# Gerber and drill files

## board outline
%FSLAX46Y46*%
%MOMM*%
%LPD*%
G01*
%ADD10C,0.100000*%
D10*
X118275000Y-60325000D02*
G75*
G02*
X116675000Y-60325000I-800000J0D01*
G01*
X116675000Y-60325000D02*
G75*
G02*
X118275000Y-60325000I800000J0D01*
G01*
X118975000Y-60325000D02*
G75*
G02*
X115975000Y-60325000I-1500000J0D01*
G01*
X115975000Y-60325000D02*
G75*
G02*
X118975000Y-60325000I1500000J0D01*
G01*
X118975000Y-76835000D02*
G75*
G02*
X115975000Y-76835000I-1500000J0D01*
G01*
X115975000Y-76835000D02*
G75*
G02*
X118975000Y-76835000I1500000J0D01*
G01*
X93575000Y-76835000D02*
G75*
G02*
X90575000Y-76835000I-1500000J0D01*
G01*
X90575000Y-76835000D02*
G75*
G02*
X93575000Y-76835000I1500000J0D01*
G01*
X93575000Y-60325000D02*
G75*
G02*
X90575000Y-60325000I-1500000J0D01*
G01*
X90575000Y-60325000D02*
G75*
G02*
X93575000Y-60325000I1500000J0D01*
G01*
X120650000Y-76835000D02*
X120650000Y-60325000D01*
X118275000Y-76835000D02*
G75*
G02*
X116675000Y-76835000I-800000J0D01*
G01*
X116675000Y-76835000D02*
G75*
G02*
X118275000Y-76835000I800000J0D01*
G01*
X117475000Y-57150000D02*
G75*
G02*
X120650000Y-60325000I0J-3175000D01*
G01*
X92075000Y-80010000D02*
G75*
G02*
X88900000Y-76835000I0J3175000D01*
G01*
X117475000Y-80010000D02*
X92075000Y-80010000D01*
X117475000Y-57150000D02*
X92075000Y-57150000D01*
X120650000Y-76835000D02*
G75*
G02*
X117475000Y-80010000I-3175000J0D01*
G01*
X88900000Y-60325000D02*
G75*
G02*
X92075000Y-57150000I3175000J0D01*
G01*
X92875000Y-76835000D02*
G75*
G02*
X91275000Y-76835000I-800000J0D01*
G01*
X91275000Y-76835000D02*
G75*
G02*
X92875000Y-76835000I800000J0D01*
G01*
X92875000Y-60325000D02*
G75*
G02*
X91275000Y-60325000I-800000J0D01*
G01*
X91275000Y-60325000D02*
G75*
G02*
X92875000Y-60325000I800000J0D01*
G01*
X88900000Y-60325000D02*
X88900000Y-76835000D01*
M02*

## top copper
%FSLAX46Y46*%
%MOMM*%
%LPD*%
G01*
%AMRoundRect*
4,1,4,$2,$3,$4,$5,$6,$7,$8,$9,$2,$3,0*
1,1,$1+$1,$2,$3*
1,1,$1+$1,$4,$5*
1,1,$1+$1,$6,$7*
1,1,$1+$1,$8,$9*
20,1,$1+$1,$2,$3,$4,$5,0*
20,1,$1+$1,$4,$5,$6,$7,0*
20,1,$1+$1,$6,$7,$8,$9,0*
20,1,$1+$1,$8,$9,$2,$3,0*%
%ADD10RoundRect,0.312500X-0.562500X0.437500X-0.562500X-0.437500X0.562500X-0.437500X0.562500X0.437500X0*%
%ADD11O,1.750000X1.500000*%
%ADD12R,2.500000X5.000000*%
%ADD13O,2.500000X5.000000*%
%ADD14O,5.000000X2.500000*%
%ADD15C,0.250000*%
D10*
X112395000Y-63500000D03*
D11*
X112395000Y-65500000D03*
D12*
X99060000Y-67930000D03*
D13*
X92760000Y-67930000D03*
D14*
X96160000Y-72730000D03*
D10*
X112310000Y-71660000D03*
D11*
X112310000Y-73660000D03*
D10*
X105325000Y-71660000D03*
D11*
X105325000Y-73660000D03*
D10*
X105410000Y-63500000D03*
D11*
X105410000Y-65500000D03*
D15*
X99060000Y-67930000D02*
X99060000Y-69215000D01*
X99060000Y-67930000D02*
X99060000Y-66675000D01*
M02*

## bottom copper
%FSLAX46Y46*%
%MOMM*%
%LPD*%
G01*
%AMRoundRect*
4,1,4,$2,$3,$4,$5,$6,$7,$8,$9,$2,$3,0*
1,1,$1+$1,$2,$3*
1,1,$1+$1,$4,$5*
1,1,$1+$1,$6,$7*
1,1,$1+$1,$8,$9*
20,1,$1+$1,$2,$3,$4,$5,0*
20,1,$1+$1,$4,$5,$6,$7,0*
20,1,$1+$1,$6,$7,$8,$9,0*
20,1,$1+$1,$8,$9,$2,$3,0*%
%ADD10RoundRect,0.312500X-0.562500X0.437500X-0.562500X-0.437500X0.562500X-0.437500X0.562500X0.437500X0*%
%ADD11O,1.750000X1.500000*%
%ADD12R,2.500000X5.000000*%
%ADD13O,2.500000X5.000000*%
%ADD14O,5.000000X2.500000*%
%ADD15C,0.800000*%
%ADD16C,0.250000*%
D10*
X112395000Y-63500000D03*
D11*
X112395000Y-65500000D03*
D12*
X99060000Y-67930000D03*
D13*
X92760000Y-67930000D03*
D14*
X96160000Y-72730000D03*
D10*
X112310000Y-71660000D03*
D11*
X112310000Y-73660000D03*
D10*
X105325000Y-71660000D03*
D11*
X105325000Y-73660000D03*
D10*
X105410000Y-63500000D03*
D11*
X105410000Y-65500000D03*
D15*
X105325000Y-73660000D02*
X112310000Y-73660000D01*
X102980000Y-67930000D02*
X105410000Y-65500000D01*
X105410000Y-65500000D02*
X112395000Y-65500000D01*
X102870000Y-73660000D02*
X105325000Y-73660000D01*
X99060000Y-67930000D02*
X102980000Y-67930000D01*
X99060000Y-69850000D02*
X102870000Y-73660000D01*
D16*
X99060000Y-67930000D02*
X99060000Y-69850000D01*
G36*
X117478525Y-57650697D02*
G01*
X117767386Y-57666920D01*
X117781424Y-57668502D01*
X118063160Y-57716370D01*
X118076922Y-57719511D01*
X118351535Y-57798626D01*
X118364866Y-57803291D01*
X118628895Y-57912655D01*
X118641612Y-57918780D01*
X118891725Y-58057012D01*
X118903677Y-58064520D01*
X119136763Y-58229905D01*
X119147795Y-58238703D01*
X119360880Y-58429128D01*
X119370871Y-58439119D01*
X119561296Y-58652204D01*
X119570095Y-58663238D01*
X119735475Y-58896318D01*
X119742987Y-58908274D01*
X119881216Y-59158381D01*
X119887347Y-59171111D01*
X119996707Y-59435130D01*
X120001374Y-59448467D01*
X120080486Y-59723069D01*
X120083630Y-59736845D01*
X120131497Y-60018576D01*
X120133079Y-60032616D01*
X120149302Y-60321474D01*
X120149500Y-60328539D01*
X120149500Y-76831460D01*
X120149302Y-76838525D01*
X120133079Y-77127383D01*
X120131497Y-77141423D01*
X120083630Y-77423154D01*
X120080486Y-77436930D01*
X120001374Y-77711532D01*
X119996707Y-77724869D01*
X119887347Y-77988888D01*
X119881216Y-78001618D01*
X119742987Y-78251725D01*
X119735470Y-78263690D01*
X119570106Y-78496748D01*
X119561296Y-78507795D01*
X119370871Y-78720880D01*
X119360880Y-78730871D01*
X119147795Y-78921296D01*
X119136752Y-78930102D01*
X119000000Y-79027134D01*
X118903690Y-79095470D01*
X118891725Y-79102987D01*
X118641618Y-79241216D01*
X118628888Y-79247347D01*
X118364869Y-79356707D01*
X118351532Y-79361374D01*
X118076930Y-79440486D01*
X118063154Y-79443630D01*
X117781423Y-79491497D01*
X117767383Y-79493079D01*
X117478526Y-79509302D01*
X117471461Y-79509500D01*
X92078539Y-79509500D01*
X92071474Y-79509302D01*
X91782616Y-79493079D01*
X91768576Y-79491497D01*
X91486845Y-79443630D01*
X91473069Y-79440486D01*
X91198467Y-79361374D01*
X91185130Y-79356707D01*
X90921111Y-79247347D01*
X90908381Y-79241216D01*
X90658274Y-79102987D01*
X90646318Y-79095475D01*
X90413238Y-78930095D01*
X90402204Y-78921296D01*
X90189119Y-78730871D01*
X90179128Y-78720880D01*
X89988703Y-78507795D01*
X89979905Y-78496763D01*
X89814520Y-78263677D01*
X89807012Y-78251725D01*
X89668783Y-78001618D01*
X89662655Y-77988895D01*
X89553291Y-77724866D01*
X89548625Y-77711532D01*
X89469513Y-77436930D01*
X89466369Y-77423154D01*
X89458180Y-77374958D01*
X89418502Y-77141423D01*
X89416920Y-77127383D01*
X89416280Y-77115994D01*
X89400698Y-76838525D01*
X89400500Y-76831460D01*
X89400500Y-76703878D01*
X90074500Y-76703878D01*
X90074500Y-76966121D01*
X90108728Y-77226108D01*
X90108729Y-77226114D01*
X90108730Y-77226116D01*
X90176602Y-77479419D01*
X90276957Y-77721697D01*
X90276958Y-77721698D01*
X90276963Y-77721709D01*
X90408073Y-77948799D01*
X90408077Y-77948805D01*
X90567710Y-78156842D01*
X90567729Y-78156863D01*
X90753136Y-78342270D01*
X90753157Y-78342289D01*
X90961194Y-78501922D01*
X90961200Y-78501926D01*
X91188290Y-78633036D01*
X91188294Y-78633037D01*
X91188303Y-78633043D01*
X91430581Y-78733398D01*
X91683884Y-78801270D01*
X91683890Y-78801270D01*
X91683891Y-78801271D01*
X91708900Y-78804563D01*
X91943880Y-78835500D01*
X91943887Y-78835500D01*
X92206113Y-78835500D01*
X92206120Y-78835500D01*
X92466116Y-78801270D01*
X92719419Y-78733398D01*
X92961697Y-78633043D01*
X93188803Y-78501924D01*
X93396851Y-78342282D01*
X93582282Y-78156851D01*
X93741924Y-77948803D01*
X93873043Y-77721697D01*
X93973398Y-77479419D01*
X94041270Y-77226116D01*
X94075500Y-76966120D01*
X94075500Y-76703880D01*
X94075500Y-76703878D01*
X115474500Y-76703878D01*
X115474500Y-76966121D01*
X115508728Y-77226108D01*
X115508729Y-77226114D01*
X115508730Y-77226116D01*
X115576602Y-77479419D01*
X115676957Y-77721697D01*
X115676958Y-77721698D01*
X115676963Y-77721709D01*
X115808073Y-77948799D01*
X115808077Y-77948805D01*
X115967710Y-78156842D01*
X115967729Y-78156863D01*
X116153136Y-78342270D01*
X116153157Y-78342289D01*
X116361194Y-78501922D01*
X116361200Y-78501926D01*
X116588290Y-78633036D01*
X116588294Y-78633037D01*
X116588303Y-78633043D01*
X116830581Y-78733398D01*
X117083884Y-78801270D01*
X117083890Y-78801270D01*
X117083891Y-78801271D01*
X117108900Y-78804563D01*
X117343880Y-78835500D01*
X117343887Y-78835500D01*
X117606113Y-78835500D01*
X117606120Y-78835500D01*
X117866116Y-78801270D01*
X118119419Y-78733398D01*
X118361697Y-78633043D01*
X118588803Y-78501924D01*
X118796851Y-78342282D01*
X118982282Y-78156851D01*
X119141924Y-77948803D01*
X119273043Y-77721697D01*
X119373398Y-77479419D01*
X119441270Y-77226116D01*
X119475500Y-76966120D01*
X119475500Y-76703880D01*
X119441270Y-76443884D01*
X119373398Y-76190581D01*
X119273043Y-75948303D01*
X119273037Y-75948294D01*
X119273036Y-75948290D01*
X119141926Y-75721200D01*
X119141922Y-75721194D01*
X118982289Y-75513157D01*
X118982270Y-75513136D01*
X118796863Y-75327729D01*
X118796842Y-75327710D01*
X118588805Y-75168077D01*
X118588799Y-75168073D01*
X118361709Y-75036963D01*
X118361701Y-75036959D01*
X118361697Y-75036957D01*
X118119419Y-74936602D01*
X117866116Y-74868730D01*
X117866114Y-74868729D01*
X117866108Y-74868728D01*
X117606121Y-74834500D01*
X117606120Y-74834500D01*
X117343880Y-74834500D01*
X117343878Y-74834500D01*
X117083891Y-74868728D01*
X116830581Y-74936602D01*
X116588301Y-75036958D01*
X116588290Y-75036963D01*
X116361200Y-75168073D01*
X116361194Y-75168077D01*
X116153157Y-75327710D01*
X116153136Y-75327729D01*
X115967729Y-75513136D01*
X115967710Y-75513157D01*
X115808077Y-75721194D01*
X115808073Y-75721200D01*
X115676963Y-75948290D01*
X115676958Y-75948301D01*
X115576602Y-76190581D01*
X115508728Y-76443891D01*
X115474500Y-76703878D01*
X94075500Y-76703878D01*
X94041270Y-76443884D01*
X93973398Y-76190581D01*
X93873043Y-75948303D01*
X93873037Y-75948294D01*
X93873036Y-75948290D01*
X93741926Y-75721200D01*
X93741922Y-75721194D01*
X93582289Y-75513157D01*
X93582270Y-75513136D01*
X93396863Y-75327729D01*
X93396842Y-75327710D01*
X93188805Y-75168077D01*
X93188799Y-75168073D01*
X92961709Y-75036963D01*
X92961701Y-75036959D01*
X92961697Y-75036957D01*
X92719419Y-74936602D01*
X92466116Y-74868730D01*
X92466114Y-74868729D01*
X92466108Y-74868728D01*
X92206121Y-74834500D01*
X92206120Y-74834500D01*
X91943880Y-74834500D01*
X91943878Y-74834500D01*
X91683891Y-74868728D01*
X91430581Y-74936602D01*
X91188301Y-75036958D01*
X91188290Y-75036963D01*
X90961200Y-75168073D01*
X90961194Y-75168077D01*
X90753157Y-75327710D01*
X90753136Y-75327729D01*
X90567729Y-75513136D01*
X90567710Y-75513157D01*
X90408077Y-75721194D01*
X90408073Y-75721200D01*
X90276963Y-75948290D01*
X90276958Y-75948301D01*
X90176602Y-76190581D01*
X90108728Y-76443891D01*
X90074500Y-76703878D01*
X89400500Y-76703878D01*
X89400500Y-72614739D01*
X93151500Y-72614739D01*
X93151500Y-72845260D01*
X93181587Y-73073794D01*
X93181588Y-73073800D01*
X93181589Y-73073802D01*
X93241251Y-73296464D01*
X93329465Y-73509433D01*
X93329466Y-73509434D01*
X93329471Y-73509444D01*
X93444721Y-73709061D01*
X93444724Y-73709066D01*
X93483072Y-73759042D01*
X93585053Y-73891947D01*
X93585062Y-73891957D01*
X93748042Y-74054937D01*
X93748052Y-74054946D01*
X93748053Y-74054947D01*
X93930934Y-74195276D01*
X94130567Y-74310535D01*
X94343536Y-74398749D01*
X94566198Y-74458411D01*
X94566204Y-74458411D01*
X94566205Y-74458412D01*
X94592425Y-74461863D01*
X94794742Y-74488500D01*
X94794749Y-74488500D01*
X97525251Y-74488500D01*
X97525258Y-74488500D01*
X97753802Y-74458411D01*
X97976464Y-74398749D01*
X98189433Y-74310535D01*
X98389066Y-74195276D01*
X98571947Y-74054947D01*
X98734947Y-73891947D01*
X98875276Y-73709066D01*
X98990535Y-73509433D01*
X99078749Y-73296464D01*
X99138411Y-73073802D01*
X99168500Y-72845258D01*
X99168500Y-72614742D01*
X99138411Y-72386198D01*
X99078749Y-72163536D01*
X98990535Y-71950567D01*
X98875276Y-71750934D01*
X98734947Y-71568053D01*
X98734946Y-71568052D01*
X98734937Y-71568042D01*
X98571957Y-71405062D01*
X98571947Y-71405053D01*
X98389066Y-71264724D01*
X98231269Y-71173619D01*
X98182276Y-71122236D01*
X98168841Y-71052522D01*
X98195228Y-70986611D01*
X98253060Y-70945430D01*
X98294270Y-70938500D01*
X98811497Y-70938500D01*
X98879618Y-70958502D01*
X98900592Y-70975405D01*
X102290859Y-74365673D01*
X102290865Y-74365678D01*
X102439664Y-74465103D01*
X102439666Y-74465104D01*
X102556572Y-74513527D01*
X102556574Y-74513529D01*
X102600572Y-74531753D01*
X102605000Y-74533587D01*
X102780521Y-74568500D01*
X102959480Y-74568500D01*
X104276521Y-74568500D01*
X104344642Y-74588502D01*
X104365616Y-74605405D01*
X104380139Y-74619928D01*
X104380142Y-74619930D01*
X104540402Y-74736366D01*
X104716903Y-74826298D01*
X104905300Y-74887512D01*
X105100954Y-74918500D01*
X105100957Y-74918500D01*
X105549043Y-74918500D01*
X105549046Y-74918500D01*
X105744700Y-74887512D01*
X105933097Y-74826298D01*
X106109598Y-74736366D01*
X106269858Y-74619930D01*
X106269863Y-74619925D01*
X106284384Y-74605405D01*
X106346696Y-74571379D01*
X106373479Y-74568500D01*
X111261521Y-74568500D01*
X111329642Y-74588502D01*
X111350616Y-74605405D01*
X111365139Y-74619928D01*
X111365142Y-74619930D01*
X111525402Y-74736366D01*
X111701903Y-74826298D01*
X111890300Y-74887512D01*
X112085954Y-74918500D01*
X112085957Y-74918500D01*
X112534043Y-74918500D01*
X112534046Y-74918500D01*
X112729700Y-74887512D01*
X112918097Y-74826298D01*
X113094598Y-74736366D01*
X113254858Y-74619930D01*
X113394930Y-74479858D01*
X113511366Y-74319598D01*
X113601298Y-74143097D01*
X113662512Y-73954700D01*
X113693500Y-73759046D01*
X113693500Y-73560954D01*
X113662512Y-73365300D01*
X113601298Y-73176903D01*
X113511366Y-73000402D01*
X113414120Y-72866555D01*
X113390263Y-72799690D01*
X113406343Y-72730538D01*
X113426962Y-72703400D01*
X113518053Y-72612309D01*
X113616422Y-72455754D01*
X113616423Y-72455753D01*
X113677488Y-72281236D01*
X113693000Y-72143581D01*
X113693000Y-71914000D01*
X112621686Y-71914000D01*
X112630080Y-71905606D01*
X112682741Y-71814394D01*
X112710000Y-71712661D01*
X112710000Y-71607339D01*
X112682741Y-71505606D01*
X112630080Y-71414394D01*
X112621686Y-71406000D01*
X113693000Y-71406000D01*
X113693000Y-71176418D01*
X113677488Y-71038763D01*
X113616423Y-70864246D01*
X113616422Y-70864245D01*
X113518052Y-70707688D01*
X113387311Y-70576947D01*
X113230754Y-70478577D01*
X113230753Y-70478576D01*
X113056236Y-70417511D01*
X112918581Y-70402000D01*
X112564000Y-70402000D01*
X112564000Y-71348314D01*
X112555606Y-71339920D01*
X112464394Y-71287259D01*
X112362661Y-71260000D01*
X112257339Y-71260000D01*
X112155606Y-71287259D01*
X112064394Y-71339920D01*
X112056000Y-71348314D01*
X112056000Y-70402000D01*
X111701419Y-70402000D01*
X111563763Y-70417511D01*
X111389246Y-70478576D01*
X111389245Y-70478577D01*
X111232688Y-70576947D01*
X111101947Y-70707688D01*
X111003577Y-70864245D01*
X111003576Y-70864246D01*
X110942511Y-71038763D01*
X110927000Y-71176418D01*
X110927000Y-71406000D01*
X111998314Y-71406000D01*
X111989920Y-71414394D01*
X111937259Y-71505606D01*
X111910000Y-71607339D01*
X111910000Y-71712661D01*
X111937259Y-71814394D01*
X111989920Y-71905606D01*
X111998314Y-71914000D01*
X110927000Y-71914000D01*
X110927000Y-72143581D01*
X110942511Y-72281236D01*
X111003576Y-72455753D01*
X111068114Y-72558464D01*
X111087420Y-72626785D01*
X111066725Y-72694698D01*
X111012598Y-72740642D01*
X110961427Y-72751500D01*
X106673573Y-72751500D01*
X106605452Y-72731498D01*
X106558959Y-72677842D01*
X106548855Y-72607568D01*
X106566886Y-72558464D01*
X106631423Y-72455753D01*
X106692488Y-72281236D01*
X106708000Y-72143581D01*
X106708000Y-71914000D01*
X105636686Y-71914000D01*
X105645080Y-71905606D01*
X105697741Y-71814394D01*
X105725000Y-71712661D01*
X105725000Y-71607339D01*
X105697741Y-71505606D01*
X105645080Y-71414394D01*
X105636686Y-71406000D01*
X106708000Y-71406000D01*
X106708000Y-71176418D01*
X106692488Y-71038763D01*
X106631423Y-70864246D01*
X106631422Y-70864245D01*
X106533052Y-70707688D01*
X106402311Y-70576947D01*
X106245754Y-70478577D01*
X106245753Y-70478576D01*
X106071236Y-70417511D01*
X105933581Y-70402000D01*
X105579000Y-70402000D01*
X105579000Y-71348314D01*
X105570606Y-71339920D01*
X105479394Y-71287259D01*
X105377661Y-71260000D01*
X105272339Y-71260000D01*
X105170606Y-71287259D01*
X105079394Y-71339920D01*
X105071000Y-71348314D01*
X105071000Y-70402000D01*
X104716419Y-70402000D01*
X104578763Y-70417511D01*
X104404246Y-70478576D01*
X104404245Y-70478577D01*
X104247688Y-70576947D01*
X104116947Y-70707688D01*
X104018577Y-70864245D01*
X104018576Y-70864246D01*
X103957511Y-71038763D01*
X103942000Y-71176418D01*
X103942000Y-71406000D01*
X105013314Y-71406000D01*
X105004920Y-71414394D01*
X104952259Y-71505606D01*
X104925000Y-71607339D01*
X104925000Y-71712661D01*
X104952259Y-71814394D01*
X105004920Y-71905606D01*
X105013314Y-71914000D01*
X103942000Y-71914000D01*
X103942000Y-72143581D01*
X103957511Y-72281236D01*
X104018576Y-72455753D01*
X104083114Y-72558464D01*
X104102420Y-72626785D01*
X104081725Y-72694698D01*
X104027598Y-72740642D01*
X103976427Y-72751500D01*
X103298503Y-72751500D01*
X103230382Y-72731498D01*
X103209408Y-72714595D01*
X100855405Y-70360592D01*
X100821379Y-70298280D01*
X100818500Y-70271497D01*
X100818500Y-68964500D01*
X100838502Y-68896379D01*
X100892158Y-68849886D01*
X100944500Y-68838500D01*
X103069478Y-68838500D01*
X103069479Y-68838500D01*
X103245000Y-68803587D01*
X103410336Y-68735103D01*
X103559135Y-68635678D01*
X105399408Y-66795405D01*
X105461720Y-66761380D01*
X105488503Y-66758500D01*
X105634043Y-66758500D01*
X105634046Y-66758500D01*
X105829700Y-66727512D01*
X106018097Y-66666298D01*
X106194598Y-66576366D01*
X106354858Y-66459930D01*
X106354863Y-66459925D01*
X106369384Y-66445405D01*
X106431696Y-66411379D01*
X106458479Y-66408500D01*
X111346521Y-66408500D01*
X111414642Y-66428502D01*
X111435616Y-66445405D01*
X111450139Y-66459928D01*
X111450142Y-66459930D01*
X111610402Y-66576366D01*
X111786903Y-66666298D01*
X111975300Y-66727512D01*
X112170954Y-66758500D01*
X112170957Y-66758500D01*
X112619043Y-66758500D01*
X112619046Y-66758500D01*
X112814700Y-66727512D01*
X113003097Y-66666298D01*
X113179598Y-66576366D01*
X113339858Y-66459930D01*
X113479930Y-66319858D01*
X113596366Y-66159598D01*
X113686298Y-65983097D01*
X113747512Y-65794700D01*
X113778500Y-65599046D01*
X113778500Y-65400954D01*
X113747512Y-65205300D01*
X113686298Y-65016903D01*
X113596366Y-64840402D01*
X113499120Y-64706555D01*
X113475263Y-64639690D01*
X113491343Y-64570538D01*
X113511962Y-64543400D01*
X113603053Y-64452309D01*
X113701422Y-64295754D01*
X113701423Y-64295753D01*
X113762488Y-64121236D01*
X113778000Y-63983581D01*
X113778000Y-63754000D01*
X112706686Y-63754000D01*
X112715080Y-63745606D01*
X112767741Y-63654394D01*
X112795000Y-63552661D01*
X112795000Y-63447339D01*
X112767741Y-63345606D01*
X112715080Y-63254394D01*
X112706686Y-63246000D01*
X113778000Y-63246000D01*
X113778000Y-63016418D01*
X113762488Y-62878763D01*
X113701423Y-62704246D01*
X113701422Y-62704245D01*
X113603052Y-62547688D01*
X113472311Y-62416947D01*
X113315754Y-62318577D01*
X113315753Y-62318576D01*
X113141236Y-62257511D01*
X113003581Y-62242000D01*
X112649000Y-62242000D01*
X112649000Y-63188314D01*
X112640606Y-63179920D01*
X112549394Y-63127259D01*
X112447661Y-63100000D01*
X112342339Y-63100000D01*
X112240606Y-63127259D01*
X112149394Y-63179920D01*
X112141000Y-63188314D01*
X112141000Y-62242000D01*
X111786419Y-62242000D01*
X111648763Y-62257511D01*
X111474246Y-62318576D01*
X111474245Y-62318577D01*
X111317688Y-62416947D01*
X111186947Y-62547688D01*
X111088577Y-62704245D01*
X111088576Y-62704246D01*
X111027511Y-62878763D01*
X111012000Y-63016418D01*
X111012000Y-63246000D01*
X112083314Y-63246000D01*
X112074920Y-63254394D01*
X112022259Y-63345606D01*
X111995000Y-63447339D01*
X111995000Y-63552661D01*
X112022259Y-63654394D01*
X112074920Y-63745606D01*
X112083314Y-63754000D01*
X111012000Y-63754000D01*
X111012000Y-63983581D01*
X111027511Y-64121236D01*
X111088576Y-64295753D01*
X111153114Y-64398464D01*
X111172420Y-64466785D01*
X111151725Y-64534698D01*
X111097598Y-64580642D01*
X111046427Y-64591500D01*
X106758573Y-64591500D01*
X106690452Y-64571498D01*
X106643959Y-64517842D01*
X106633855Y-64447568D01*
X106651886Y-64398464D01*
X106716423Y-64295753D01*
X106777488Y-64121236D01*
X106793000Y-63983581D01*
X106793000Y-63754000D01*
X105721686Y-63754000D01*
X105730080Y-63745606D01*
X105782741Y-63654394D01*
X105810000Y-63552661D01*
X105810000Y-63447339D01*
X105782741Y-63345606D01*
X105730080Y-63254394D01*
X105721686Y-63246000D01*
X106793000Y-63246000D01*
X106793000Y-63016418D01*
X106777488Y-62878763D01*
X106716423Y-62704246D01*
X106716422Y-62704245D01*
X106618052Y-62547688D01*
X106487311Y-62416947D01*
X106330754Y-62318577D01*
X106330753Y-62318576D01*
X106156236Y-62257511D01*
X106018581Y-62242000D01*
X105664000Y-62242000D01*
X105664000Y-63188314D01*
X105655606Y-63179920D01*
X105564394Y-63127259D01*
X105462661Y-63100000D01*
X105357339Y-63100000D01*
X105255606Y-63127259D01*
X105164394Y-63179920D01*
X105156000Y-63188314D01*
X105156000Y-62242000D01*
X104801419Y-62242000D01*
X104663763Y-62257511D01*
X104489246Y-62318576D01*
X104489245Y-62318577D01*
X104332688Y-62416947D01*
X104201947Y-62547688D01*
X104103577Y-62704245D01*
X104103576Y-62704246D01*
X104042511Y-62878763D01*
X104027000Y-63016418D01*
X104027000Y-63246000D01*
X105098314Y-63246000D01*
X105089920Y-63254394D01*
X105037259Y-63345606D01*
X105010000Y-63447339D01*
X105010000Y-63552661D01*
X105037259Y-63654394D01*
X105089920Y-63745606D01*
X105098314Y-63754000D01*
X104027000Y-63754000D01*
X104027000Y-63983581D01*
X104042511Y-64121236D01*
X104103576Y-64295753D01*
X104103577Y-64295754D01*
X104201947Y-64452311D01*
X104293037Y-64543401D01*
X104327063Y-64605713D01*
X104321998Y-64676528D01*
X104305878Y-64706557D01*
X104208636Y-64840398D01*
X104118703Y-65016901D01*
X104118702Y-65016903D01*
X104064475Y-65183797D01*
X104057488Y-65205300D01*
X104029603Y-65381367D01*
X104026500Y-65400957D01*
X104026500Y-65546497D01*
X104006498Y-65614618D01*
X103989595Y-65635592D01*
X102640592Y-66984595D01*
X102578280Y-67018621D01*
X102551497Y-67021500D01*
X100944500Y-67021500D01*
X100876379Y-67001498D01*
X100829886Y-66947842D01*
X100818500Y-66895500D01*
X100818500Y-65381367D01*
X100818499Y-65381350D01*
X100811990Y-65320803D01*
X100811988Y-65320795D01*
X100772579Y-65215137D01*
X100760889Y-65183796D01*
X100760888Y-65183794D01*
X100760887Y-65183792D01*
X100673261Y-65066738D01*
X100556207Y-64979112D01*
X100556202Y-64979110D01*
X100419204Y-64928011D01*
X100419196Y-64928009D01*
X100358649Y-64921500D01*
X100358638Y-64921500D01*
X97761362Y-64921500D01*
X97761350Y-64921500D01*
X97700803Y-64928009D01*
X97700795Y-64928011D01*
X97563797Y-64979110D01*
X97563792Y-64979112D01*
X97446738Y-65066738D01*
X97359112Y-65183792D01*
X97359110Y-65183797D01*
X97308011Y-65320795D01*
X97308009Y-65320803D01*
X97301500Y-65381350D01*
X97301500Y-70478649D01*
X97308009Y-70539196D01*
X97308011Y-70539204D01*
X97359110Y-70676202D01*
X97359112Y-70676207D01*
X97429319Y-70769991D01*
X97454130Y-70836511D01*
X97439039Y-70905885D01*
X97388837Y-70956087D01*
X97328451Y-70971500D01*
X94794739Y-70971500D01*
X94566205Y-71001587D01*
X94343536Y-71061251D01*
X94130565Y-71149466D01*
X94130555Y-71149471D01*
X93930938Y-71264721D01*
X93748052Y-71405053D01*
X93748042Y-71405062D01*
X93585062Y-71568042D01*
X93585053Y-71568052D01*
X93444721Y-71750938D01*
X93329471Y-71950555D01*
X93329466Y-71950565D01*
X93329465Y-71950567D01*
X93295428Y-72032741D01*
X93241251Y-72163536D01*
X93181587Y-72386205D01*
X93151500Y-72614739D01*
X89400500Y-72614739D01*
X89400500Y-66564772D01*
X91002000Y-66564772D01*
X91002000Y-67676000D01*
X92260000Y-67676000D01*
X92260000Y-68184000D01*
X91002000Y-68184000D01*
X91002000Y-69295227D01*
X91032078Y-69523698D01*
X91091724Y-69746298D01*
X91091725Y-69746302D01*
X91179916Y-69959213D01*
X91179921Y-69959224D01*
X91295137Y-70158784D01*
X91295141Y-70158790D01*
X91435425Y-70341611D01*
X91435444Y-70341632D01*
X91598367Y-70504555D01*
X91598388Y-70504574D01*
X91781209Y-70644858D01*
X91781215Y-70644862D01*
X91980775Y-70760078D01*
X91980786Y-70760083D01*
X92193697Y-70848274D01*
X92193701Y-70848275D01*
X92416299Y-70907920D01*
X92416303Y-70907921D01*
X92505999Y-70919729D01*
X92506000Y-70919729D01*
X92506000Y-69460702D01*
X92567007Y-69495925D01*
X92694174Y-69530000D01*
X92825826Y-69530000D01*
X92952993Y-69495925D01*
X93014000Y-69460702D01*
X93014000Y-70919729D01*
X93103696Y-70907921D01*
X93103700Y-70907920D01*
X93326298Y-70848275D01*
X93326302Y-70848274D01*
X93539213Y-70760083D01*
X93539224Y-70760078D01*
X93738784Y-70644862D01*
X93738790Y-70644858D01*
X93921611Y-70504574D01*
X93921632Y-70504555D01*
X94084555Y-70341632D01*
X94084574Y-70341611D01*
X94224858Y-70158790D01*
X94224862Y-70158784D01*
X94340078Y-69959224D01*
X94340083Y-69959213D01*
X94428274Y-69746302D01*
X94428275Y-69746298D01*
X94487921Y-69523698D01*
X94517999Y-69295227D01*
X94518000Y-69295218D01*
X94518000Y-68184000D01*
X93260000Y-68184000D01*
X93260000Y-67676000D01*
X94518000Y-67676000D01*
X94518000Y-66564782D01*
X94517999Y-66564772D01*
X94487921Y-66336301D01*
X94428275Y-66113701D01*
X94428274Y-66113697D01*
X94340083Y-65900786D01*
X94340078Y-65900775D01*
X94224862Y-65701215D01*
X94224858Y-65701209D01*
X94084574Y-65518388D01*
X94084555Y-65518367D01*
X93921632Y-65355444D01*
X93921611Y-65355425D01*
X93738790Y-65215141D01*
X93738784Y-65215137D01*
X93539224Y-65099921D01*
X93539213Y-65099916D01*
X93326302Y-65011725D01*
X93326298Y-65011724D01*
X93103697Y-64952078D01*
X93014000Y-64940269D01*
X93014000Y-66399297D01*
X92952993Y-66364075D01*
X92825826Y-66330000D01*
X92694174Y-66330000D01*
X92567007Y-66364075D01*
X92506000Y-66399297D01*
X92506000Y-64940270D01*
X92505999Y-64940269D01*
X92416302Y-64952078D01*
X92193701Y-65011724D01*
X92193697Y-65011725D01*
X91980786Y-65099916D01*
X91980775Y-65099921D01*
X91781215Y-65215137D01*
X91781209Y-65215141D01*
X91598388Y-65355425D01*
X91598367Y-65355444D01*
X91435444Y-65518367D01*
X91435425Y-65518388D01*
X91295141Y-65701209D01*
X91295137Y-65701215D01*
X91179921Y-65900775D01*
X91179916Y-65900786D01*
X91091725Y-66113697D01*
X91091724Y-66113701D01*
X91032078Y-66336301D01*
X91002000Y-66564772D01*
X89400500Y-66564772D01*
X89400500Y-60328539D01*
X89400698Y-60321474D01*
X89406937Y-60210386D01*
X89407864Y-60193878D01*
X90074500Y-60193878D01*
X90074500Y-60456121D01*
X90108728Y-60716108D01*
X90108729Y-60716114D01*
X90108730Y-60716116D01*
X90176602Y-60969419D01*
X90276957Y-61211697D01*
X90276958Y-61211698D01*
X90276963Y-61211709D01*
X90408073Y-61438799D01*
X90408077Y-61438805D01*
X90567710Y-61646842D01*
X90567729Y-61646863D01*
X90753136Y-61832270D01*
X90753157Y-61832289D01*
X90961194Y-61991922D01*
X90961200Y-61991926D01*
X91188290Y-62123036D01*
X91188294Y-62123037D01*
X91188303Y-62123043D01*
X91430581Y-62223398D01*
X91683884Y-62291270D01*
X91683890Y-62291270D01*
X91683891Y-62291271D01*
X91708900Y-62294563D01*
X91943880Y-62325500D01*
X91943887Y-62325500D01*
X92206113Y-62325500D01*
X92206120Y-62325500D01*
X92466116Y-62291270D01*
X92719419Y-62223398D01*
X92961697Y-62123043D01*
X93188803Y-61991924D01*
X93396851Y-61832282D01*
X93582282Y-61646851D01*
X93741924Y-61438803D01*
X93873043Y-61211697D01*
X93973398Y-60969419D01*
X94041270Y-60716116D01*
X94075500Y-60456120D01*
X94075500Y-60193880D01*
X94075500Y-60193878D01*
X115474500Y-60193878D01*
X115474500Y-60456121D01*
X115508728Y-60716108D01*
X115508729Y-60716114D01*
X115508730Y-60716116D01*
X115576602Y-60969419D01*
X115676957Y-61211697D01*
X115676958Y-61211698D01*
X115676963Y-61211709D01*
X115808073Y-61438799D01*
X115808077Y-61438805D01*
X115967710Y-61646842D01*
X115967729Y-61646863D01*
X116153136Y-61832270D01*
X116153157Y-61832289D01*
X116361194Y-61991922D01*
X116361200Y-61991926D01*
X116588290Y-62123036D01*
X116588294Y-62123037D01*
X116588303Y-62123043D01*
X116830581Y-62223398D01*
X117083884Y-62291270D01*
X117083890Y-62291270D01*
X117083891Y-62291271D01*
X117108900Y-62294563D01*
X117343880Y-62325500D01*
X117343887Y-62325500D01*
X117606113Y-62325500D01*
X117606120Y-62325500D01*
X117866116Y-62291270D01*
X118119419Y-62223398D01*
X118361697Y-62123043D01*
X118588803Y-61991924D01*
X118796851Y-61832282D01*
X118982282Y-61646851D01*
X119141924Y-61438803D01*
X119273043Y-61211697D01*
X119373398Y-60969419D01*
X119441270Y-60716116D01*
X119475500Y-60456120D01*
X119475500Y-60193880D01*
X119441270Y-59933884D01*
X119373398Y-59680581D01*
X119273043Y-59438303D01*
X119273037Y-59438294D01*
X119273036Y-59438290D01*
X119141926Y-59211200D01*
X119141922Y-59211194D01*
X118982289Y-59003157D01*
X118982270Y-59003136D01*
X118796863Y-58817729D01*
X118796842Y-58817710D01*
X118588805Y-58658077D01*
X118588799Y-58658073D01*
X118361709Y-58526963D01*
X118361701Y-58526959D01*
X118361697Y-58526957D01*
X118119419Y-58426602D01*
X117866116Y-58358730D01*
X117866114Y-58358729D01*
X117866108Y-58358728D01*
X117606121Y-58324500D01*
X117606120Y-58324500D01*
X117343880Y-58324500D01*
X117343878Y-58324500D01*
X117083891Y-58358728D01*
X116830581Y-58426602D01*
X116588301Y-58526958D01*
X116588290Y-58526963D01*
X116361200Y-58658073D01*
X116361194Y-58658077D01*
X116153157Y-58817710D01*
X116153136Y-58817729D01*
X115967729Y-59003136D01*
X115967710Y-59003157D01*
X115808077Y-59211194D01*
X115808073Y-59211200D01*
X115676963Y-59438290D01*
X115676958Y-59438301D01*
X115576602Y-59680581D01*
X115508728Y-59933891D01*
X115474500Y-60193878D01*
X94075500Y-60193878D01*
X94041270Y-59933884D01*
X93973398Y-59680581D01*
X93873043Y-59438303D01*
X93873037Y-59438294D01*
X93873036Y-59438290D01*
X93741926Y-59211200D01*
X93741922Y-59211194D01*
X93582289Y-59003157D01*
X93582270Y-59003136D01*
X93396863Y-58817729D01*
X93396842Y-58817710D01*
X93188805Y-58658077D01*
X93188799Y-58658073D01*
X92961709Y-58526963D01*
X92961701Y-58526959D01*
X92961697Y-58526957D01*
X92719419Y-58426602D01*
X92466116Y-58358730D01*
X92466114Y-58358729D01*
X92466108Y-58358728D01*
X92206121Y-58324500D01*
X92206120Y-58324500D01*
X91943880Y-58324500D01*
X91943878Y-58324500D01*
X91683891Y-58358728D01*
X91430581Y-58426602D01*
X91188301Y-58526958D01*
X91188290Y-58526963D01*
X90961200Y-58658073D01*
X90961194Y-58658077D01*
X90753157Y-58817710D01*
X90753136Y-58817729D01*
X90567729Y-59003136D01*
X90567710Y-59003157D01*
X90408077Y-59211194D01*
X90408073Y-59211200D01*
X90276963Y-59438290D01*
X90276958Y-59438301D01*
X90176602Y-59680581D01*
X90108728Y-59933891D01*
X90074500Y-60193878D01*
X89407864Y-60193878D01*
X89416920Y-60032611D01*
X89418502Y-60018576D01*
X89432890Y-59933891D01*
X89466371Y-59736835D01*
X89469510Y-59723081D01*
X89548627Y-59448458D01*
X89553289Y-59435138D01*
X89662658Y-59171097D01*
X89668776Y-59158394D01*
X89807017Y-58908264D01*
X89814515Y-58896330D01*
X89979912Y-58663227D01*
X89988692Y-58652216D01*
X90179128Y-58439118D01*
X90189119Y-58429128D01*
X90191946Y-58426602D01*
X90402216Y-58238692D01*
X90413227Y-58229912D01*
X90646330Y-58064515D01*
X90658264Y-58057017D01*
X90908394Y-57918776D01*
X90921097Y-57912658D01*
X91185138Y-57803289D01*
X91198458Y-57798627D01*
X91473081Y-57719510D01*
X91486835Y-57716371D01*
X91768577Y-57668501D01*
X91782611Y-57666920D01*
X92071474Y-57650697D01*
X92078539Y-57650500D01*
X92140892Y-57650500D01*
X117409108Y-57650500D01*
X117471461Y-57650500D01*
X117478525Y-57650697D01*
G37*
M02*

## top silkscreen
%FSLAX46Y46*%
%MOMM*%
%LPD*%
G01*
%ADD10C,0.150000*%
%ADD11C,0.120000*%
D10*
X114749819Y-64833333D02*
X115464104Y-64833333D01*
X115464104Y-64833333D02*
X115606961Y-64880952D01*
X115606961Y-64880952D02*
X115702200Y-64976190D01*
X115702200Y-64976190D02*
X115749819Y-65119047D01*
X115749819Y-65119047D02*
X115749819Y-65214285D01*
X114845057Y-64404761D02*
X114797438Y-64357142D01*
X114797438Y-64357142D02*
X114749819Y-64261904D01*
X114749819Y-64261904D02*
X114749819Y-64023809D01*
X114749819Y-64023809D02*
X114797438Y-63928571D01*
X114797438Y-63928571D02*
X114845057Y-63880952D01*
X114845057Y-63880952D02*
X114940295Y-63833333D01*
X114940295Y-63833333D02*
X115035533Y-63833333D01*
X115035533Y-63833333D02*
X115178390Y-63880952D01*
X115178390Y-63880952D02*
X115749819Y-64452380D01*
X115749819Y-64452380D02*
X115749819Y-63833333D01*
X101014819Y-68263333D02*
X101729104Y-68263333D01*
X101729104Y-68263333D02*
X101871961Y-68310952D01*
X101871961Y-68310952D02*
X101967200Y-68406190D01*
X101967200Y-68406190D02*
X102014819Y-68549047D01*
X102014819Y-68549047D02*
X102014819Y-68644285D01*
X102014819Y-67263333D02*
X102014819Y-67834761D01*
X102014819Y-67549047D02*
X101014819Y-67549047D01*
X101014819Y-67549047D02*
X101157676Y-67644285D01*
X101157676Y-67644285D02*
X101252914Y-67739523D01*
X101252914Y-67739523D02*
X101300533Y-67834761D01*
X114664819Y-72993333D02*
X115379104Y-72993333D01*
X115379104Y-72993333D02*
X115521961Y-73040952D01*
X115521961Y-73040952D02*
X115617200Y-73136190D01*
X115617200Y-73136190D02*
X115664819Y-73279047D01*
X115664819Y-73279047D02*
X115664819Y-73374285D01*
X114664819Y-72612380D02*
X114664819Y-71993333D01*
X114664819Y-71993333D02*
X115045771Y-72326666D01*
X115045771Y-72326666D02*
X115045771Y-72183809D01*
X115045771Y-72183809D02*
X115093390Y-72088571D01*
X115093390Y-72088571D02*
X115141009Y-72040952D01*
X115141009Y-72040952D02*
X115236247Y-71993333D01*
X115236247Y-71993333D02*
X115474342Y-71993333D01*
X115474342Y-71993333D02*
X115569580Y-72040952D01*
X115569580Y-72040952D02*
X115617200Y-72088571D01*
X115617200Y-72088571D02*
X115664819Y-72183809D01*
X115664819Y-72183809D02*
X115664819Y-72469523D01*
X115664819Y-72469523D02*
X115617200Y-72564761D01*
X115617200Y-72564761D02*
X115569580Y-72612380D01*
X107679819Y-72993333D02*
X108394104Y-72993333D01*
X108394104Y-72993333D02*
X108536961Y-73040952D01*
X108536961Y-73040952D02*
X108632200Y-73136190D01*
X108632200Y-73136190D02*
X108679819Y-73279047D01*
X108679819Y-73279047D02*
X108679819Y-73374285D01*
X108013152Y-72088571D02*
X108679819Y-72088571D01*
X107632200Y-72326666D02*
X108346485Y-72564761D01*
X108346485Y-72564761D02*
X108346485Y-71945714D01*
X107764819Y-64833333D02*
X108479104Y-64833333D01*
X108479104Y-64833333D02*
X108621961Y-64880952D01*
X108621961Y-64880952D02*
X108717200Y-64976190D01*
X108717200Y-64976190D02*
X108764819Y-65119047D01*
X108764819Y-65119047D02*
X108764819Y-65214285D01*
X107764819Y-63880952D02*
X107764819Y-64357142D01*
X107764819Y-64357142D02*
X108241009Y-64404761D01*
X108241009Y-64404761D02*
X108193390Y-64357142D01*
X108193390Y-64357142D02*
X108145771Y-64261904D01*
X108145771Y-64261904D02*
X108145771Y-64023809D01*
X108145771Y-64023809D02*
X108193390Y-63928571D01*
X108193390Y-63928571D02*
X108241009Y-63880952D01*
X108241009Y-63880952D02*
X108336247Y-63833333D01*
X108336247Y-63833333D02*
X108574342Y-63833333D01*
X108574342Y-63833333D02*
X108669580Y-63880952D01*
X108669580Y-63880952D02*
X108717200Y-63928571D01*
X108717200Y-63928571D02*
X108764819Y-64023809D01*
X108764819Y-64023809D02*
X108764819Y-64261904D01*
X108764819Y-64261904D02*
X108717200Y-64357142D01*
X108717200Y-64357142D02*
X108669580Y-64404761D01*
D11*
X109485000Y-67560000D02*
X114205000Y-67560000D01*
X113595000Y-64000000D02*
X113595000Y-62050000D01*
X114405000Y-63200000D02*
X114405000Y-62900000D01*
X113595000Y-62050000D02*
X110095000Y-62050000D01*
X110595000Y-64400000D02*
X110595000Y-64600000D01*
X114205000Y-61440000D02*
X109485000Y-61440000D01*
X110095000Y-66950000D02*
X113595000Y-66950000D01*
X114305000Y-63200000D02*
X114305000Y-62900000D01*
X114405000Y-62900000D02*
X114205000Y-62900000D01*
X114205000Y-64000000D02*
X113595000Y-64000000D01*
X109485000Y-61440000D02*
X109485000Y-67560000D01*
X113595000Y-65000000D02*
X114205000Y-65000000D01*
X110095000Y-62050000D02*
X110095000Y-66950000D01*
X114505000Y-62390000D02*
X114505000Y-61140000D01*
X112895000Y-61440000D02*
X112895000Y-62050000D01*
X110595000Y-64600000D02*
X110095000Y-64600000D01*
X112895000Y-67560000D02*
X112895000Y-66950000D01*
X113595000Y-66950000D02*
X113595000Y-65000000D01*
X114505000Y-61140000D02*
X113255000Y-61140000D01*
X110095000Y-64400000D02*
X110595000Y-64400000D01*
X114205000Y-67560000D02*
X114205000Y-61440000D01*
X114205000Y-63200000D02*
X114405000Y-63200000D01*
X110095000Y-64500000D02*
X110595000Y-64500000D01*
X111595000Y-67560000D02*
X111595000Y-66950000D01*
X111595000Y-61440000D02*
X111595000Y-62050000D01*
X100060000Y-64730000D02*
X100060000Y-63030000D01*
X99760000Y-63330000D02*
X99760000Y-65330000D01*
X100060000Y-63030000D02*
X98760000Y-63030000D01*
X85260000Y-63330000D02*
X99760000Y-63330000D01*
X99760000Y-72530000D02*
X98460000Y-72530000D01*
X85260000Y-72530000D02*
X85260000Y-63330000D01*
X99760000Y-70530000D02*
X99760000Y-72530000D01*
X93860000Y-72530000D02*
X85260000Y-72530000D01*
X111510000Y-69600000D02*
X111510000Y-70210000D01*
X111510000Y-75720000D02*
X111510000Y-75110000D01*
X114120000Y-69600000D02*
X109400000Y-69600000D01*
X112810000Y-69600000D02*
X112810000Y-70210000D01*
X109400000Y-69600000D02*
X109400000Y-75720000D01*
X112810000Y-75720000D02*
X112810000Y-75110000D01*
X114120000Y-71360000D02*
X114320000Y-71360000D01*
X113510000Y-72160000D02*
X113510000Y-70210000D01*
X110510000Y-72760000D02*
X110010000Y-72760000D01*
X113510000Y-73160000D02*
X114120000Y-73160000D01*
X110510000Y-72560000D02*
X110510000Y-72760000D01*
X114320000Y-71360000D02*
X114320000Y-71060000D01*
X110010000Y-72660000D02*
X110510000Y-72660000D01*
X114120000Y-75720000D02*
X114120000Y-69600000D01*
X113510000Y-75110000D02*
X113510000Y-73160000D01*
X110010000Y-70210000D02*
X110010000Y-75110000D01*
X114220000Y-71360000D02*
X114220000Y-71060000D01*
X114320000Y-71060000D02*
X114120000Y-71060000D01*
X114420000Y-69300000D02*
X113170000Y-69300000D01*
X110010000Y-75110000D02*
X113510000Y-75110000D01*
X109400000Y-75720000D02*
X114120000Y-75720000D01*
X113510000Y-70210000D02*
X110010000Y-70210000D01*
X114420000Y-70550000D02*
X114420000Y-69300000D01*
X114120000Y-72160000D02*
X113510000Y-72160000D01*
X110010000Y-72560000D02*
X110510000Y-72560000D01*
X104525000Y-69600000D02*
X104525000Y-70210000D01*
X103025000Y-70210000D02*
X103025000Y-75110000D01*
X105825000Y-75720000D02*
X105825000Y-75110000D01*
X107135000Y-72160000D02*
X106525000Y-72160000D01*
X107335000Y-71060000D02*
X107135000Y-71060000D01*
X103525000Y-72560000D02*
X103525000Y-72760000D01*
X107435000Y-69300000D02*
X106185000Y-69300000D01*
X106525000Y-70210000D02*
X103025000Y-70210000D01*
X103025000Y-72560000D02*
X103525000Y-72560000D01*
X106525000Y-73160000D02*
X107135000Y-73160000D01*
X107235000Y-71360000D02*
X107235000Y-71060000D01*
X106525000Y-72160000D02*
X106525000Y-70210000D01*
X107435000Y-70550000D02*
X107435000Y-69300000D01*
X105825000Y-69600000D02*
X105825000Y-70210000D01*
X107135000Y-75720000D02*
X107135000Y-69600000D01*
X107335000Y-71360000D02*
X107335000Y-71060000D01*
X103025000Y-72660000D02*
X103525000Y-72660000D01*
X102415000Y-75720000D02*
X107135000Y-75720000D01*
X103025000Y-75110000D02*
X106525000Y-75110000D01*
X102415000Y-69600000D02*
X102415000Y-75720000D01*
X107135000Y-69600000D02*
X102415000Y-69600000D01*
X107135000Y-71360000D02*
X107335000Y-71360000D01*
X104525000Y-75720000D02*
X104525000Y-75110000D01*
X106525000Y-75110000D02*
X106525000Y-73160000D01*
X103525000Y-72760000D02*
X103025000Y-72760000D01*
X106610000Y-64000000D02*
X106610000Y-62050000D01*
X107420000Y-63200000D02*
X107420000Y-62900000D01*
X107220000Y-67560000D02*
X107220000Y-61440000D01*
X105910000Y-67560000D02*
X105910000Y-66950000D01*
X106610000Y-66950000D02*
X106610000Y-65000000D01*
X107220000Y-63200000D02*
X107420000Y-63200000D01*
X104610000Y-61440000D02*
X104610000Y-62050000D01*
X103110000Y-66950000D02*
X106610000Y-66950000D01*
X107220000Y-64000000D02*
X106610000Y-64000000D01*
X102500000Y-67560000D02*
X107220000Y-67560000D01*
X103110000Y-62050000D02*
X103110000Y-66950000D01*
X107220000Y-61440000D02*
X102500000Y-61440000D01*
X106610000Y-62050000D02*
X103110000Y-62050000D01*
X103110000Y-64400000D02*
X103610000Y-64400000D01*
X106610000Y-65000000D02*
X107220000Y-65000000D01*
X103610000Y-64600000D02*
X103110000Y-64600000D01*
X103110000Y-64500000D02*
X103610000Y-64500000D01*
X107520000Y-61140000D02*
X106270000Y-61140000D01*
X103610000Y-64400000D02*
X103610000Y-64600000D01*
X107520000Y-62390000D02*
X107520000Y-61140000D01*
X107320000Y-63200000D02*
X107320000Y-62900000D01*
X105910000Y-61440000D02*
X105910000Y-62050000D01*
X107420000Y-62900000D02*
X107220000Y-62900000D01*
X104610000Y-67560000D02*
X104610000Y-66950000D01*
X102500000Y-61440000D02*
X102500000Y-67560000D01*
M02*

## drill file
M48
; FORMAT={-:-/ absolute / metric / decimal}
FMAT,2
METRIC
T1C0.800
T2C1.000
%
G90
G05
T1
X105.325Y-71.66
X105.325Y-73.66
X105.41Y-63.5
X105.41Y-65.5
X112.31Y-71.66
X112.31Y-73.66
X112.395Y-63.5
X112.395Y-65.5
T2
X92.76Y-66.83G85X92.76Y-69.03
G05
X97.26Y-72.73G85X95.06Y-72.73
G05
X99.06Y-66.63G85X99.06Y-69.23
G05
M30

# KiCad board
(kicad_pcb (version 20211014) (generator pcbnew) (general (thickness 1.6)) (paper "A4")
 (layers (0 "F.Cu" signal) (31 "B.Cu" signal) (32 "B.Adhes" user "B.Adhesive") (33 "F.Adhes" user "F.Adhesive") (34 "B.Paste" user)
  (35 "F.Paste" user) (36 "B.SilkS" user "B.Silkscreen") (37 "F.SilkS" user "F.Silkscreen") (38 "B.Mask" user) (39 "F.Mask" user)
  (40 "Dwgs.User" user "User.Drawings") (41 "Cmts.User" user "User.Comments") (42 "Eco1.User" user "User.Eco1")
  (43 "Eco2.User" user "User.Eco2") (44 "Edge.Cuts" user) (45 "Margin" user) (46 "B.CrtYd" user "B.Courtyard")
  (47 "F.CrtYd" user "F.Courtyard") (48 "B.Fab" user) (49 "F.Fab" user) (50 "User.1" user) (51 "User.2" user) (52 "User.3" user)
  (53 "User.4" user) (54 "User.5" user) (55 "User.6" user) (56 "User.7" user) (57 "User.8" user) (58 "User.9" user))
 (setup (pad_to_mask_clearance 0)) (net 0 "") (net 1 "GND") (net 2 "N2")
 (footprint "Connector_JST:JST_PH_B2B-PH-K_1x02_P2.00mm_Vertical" (layer "F.Cu") (at 112.395 63.5 -90)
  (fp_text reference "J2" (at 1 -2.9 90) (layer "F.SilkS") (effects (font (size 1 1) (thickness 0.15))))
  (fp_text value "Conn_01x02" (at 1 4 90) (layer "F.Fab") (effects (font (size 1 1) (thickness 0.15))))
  (fp_line (start 4.06 2.91) (end 4.06 -1.81) (layer "F.SilkS") (width 0.12))
  (fp_line (start 0.5 -1.2) (end -1.45 -1.2) (layer "F.SilkS") (width 0.12))
  (fp_line (start -0.3 -2.01) (end -0.6 -2.01) (layer "F.SilkS") (width 0.12))
  (fp_line (start -1.45 -1.2) (end -1.45 2.3) (layer "F.SilkS") (width 0.12))
  (fp_line (start 0.9 1.8) (end 1.1 1.8) (layer "F.SilkS") (width 0.12))
  (fp_line (start -2.06 -1.81) (end -2.06 2.91) (layer "F.SilkS") (width 0.12))
  (fp_line (start 3.45 2.3) (end 3.45 -1.2) (layer "F.SilkS") (width 0.12))
  (fp_line (start -0.3 -1.91) (end -0.6 -1.91) (layer "F.SilkS") (width 0.12))
  (fp_line (start -0.6 -2.01) (end -0.6 -1.81) (layer "F.SilkS") (width 0.12))
  (fp_line (start 0.5 -1.81) (end 0.5 -1.2) (layer "F.SilkS") (width 0.12))
  (fp_line (start -2.06 2.91) (end 4.06 2.91) (layer "F.SilkS") (width 0.12))
  (fp_line (start 1.5 -1.2) (end 1.5 -1.81) (layer "F.SilkS") (width 0.12))
  (fp_line (start -1.45 2.3) (end 3.45 2.3) (layer "F.SilkS") (width 0.12))
  (fp_line (start -1.11 -2.11) (end -2.36 -2.11) (layer "F.SilkS") (width 0.12))
  (fp_line (start -2.06 -0.5) (end -1.45 -0.5) (layer "F.SilkS") (width 0.12))
  (fp_line (start 1.1 1.8) (end 1.1 2.3) (layer "F.SilkS") (width 0.12))
  (fp_line (start 4.06 -0.5) (end 3.45 -0.5) (layer "F.SilkS") (width 0.12))
  (fp_line (start 3.45 -1.2) (end 1.5 -1.2) (layer "F.SilkS") (width 0.12))
  (fp_line (start -2.36 -2.11) (end -2.36 -0.86) (layer "F.SilkS") (width 0.12))
  (fp_line (start 0.9 2.3) (end 0.9 1.8) (layer "F.SilkS") (width 0.12))
  (fp_line (start 4.06 -1.81) (end -2.06 -1.81) (layer "F.SilkS") (width 0.12))
  (fp_line (start -0.3 -1.81) (end -0.3 -2.01) (layer "F.SilkS") (width 0.12))
  (fp_line (start 1 2.3) (end 1 1.8) (layer "F.SilkS") (width 0.12))
  (fp_line (start 4.06 0.8) (end 3.45 0.8) (layer "F.SilkS") (width 0.12))
  (fp_line (start -2.06 0.8) (end -1.45 0.8) (layer "F.SilkS") (width 0.12))
  (pad "1" thru_hole roundrect (at 0 0 270) (size 1.5 1.75) (drill 0.8) (layers *.Cu *.Mask) (roundrect_rratio 0.208333) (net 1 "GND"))
  (pad "2" thru_hole oval (at 2 0 270) (size 1.5 1.75) (drill 0.8) (layers *.Cu *.Mask) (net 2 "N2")))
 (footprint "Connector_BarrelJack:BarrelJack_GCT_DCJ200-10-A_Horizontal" (layer "F.Cu") (at 99.06 67.93 -90)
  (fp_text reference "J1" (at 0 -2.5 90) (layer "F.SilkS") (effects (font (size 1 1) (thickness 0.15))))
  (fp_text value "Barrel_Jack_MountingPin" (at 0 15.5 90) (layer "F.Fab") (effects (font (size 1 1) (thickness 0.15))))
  (fp_line (start -3.2 -1) (end -4.9 -1) (layer "F.SilkS") (width 0.12))
  (fp_line (start -4.6 -0.7) (end -2.6 -0.7) (layer "F.SilkS") (width 0.12))
  (fp_line (start -4.9 -1) (end -4.9 0.3) (layer "F.SilkS") (width 0.12))
  (fp_line (start -4.6 13.8) (end -4.6 -0.7) (layer "F.SilkS") (width 0.12))
  (fp_line (start 4.6 -0.7) (end 4.6 0.6) (layer "F.SilkS") (width 0.12))
  (fp_line (start 4.6 13.8) (end -4.6 13.8) (layer "F.SilkS") (width 0.12))
  (fp_line (start 2.6 -0.7) (end 4.6 -0.7) (layer "F.SilkS") (width 0.12))
  (fp_line (start 4.6 5.2) (end 4.6 13.8) (layer "F.SilkS") (width 0.12))
  (pad "1" thru_hole rect (at 0 0 270) (size 5 2.5) (drill oval 3.6 1) (layers *.Cu *.Mask) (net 2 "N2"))
  (pad "2" thru_hole oval (at 0 6.3 270) (size 5 2.5) (drill oval 3.2 1) (layers *.Cu *.Mask) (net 1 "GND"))
  (pad "3" thru_hole oval (at 4.8 2.9 270) (size 2.5 5) (drill oval 1 3.2) (layers *.Cu *.Mask)))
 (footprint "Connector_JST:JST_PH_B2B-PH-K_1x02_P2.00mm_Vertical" (layer "F.Cu") (at 112.31 71.66 -90)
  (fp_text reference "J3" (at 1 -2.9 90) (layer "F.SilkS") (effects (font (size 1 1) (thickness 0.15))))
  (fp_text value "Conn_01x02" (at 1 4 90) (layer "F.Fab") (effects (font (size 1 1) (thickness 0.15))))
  (fp_line (start -2.06 0.8) (end -1.45 0.8) (layer "F.SilkS") (width 0.12))
  (fp_line (start 4.06 0.8) (end 3.45 0.8) (layer "F.SilkS") (width 0.12))
  (fp_line (start -2.06 -1.81) (end -2.06 2.91) (layer "F.SilkS") (width 0.12))
  (fp_line (start -2.06 -0.5) (end -1.45 -0.5) (layer "F.SilkS") (width 0.12))
  (fp_line (start -2.06 2.91) (end 4.06 2.91) (layer "F.SilkS") (width 0.12))
  (fp_line (start 4.06 -0.5) (end 3.45 -0.5) (layer "F.SilkS") (width 0.12))
  (fp_line (start -0.3 -1.81) (end -0.3 -2.01) (layer "F.SilkS") (width 0.12))
  (fp_line (start 0.5 -1.2) (end -1.45 -1.2) (layer "F.SilkS") (width 0.12))
  (fp_line (start 1.1 1.8) (end 1.1 2.3) (layer "F.SilkS") (width 0.12))
  (fp_line (start 1.5 -1.2) (end 1.5 -1.81) (layer "F.SilkS") (width 0.12))
  (fp_line (start 0.9 1.8) (end 1.1 1.8) (layer "F.SilkS") (width 0.12))
  (fp_line (start -0.3 -2.01) (end -0.6 -2.01) (layer "F.SilkS") (width 0.12))
  (fp_line (start 1 2.3) (end 1 1.8) (layer "F.SilkS") (width 0.12))
  (fp_line (start 4.06 -1.81) (end -2.06 -1.81) (layer "F.SilkS") (width 0.12))
  (fp_line (start 3.45 -1.2) (end 1.5 -1.2) (layer "F.SilkS") (width 0.12))
  (fp_line (start -1.45 2.3) (end 3.45 2.3) (layer "F.SilkS") (width 0.12))
  (fp_line (start -0.3 -1.91) (end -0.6 -1.91) (layer "F.SilkS") (width 0.12))
  (fp_line (start -0.6 -2.01) (end -0.6 -1.81) (layer "F.SilkS") (width 0.12))
  (fp_line (start -2.36 -2.11) (end -2.36 -0.86) (layer "F.SilkS") (width 0.12))
  (fp_line (start 3.45 2.3) (end 3.45 -1.2) (layer "F.SilkS") (width 0.12))
  (fp_line (start 4.06 2.91) (end 4.06 -1.81) (layer "F.SilkS") (width 0.12))
  (fp_line (start -1.45 -1.2) (end -1.45 2.3) (layer "F.SilkS") (width 0.12))
  (fp_line (start -1.11 -2.11) (end -2.36 -2.11) (layer "F.SilkS") (width 0.12))
  (fp_line (start 0.5 -1.81) (end 0.5 -1.2) (layer "F.SilkS") (width 0.12))
  (fp_line (start 0.9 2.3) (end 0.9 1.8) (layer "F.SilkS") (width 0.12))
  (pad "1" thru_hole roundrect (at 0 0 270) (size 1.5 1.75) (drill 0.8) (layers *.Cu *.Mask) (roundrect_rratio 0.208333) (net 1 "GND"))
  (pad "2" thru_hole oval (at 2 0 270) (size 1.5 1.75) (drill 0.8) (layers *.Cu *.Mask) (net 2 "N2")))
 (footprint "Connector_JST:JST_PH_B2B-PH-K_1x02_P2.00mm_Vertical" (layer "F.Cu") (at 105.325 71.66 -90)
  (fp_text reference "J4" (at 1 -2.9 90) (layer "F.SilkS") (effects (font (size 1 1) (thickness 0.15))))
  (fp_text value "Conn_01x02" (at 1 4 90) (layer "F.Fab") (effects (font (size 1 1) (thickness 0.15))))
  (fp_line (start -2.06 0.8) (end -1.45 0.8) (layer "F.SilkS") (width 0.12))
  (fp_line (start -1.45 2.3) (end 3.45 2.3) (layer "F.SilkS") (width 0.12))
  (fp_line (start 4.06 -0.5) (end 3.45 -0.5) (layer "F.SilkS") (width 0.12))
  (fp_line (start 0.5 -1.81) (end 0.5 -1.2) (layer "F.SilkS") (width 0.12))
  (fp_line (start -0.6 -2.01) (end -0.6 -1.81) (layer "F.SilkS") (width 0.12))
  (fp_line (start 0.9 1.8) (end 1.1 1.8) (layer "F.SilkS") (width 0.12))
  (fp_line (start -2.36 -2.11) (end -2.36 -0.86) (layer "F.SilkS") (width 0.12))
  (fp_line (start -1.45 -1.2) (end -1.45 2.3) (layer "F.SilkS") (width 0.12))
  (fp_line (start 0.9 2.3) (end 0.9 1.8) (layer "F.SilkS") (width 0.12))
  (fp_line (start 1.5 -1.2) (end 1.5 -1.81) (layer "F.SilkS") (width 0.12))
  (fp_line (start -0.3 -1.91) (end -0.6 -1.91) (layer "F.SilkS") (width 0.12))
  (fp_line (start 0.5 -1.2) (end -1.45 -1.2) (layer "F.SilkS") (width 0.12))
  (fp_line (start -1.11 -2.11) (end -2.36 -2.11) (layer "F.SilkS") (width 0.12))
  (fp_line (start -2.06 -0.5) (end -1.45 -0.5) (layer "F.SilkS") (width 0.12))
  (fp_line (start 4.06 -1.81) (end -2.06 -1.81) (layer "F.SilkS") (width 0.12))
  (fp_line (start -0.3 -2.01) (end -0.6 -2.01) (layer "F.SilkS") (width 0.12))
  (fp_line (start 1 2.3) (end 1 1.8) (layer "F.SilkS") (width 0.12))
  (fp_line (start 4.06 2.91) (end 4.06 -1.81) (layer "F.SilkS") (width 0.12))
  (fp_line (start 3.45 2.3) (end 3.45 -1.2) (layer "F.SilkS") (width 0.12))
  (fp_line (start -2.06 2.91) (end 4.06 2.91) (layer "F.SilkS") (width 0.12))
  (fp_line (start -2.06 -1.81) (end -2.06 2.91) (layer "F.SilkS") (width 0.12))
  (fp_line (start -0.3 -1.81) (end -0.3 -2.01) (layer "F.SilkS") (width 0.12))
  (fp_line (start 4.06 0.8) (end 3.45 0.8) (layer "F.SilkS") (width 0.12))
  (fp_line (start 3.45 -1.2) (end 1.5 -1.2) (layer "F.SilkS") (width 0.12))
  (fp_line (start 1.1 1.8) (end 1.1 2.3) (layer "F.SilkS") (width 0.12))
  (pad "1" thru_hole roundrect (at 0 0 270) (size 1.5 1.75) (drill 0.8) (layers *.Cu *.Mask) (roundrect_rratio 0.208333) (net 1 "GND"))
  (pad "2" thru_hole oval (at 2 0 270) (size 1.5 1.75) (drill 0.8) (layers *.Cu *.Mask) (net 2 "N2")))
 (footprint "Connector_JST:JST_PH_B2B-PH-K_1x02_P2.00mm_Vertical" (layer "F.Cu") (at 105.41 63.5 -90)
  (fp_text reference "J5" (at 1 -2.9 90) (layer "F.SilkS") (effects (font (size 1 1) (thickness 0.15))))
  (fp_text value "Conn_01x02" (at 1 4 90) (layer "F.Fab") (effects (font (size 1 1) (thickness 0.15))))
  (fp_line (start 0.5 -1.2) (end -1.45 -1.2) (layer "F.SilkS") (width 0.12))
  (fp_line (start -0.3 -2.01) (end -0.6 -2.01) (layer "F.SilkS") (width 0.12))
  (fp_line (start 4.06 -1.81) (end -2.06 -1.81) (layer "F.SilkS") (width 0.12))
  (fp_line (start 4.06 -0.5) (end 3.45 -0.5) (layer "F.SilkS") (width 0.12))
  (fp_line (start 3.45 -1.2) (end 1.5 -1.2) (layer "F.SilkS") (width 0.12))
  (fp_line (start -0.3 -1.81) (end -0.3 -2.01) (layer "F.SilkS") (width 0.12))
  (fp_line (start -2.06 0.8) (end -1.45 0.8) (layer "F.SilkS") (width 0.12))
  (fp_line (start 3.45 2.3) (end 3.45 -1.2) (layer "F.SilkS") (width 0.12))
  (fp_line (start 0.5 -1.81) (end 0.5 -1.2) (layer "F.SilkS") (width 0.12))
  (fp_line (start 4.06 2.91) (end 4.06 -1.81) (layer "F.SilkS") (width 0.12))
  (fp_line (start -1.45 2.3) (end 3.45 2.3) (layer "F.SilkS") (width 0.12))
  (fp_line (start -2.06 -1.81) (end -2.06 2.91) (layer "F.SilkS") (width 0.12))
  (fp_line (start -1.45 -1.2) (end -1.45 2.3) (layer "F.SilkS") (width 0.12))
  (fp_line (start 0.9 2.3) (end 0.9 1.8) (layer "F.SilkS") (width 0.12))
  (fp_line (start 1.5 -1.2) (end 1.5 -1.81) (layer "F.SilkS") (width 0.12))
  (fp_line (start 1.1 1.8) (end 1.1 2.3) (layer "F.SilkS") (width 0.12))
  (fp_line (start 1 2.3) (end 1 1.8) (layer "F.SilkS") (width 0.12))
  (fp_line (start -2.36 -2.11) (end -2.36 -0.86) (layer "F.SilkS") (width 0.12))
  (fp_line (start 0.9 1.8) (end 1.1 1.8) (layer "F.SilkS") (width 0.12))
  (fp_line (start -1.11 -2.11) (end -2.36 -2.11) (layer "F.SilkS") (width 0.12))
  (fp_line (start -0.3 -1.91) (end -0.6 -1.91) (layer "F.SilkS") (width 0.12))
  (fp_line (start -2.06 -0.5) (end -1.45 -0.5) (layer "F.SilkS") (width 0.12))
  (fp_line (start -0.6 -2.01) (end -0.6 -1.81) (layer "F.SilkS") (width 0.12))
  (fp_line (start 4.06 0.8) (end 3.45 0.8) (layer "F.SilkS") (width 0.12))
  (fp_line (start -2.06 2.91) (end 4.06 2.91) (layer "F.SilkS") (width 0.12))
  (pad "1" thru_hole roundrect (at 0 0 270) (size 1.5 1.75) (drill 0.8) (layers *.Cu *.Mask) (roundrect_rratio 0.208333) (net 1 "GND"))
  (pad "2" thru_hole oval (at 2 0 270) (size 1.5 1.75) (drill 0.8) (layers *.Cu *.Mask) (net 2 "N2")))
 (gr_circle (center 117.475 60.325) (end 118.275 60.325) (layer "Edge.Cuts") (width 0.1) (fill none))
 (gr_circle (center 117.475 60.325) (end 118.975 60.325) (layer "Edge.Cuts") (width 0.1) (fill none))
 (gr_circle (center 117.475 76.835) (end 118.975 76.835) (layer "Edge.Cuts") (width 0.1) (fill none))
 (gr_circle (center 92.075 76.835) (end 93.575 76.835) (layer "Edge.Cuts") (width 0.1) (fill none))
 (gr_circle (center 92.075 60.325) (end 93.575 60.325) (layer "Edge.Cuts") (width 0.1) (fill none))
 (gr_line (start 120.65 76.835) (end 120.65 60.325) (layer "Edge.Cuts") (width 0.1))
 (gr_circle (center 117.475 76.835) (end 118.275 76.835) (layer "Edge.Cuts") (width 0.1) (fill none))
 (gr_arc (start 117.475 57.15) (mid 119.720064 58.079936) (end 120.65 60.325) (layer "Edge.Cuts") (width 0.1))
 (gr_arc (start 92.075 80.01) (mid 89.829936 79.080064) (end 88.9 76.835) (layer "Edge.Cuts") (width 0.1))
 (gr_line (start 117.475 80.01) (end 92.075 80.01) (layer "Edge.Cuts") (width 0.1))
 (gr_line (start 117.475 57.15) (end 92.075 57.15) (layer "Edge.Cuts") (width 0.1))
 (gr_arc (start 120.65 76.835) (mid 119.720064 79.080064) (end 117.475 80.01) (layer "Edge.Cuts") (width 0.1))
 (gr_arc (start 88.9 60.325) (mid 89.829936 58.079936) (end 92.075 57.15) (layer "Edge.Cuts") (width 0.1))
 (gr_circle (center 92.075 76.835) (end 92.875 76.835) (layer "Edge.Cuts") (width 0.1) (fill none))
 (gr_circle (center 92.075 60.325) (end 92.875 60.325) (layer "Edge.Cuts") (width 0.1) (fill none))
 (gr_line (start 88.9 60.325) (end 88.9 76.835) (layer "Edge.Cuts") (width 0.1))
 (segment (start 99.06 67.93) (end 99.06 69.215) (width 0.25) (layer "F.Cu") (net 2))
 (segment (start 99.06 67.93) (end 99.06 66.675) (width 0.25) (layer "F.Cu") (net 2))
 (segment (start 105.325 73.66) (end 112.31 73.66) (width 0.8) (layer "B.Cu") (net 2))
 (segment (start 102.98 67.93) (end 105.41 65.5) (width 0.8) (layer "B.Cu") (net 2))
 (segment (start 105.41 65.5) (end 112.395 65.5) (width 0.8) (layer "B.Cu") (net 2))
 (segment (start 102.87 73.66) (end 105.325 73.66) (width 0.8) (layer "B.Cu") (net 2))
 (segment (start 99.06 67.93) (end 102.98 67.93) (width 0.8) (layer "B.Cu") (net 2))
 (segment (start 99.06 69.85) (end 102.87 73.66) (width 0.8) (layer "B.Cu") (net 2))
 (segment (start 99.06 67.93) (end 99.06 69.85) (width 0.25) (layer "B.Cu") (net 2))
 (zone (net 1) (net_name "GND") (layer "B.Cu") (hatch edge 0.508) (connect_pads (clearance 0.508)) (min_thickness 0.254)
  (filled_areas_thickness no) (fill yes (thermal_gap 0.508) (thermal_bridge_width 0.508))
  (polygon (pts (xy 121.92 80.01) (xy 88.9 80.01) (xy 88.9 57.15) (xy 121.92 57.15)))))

